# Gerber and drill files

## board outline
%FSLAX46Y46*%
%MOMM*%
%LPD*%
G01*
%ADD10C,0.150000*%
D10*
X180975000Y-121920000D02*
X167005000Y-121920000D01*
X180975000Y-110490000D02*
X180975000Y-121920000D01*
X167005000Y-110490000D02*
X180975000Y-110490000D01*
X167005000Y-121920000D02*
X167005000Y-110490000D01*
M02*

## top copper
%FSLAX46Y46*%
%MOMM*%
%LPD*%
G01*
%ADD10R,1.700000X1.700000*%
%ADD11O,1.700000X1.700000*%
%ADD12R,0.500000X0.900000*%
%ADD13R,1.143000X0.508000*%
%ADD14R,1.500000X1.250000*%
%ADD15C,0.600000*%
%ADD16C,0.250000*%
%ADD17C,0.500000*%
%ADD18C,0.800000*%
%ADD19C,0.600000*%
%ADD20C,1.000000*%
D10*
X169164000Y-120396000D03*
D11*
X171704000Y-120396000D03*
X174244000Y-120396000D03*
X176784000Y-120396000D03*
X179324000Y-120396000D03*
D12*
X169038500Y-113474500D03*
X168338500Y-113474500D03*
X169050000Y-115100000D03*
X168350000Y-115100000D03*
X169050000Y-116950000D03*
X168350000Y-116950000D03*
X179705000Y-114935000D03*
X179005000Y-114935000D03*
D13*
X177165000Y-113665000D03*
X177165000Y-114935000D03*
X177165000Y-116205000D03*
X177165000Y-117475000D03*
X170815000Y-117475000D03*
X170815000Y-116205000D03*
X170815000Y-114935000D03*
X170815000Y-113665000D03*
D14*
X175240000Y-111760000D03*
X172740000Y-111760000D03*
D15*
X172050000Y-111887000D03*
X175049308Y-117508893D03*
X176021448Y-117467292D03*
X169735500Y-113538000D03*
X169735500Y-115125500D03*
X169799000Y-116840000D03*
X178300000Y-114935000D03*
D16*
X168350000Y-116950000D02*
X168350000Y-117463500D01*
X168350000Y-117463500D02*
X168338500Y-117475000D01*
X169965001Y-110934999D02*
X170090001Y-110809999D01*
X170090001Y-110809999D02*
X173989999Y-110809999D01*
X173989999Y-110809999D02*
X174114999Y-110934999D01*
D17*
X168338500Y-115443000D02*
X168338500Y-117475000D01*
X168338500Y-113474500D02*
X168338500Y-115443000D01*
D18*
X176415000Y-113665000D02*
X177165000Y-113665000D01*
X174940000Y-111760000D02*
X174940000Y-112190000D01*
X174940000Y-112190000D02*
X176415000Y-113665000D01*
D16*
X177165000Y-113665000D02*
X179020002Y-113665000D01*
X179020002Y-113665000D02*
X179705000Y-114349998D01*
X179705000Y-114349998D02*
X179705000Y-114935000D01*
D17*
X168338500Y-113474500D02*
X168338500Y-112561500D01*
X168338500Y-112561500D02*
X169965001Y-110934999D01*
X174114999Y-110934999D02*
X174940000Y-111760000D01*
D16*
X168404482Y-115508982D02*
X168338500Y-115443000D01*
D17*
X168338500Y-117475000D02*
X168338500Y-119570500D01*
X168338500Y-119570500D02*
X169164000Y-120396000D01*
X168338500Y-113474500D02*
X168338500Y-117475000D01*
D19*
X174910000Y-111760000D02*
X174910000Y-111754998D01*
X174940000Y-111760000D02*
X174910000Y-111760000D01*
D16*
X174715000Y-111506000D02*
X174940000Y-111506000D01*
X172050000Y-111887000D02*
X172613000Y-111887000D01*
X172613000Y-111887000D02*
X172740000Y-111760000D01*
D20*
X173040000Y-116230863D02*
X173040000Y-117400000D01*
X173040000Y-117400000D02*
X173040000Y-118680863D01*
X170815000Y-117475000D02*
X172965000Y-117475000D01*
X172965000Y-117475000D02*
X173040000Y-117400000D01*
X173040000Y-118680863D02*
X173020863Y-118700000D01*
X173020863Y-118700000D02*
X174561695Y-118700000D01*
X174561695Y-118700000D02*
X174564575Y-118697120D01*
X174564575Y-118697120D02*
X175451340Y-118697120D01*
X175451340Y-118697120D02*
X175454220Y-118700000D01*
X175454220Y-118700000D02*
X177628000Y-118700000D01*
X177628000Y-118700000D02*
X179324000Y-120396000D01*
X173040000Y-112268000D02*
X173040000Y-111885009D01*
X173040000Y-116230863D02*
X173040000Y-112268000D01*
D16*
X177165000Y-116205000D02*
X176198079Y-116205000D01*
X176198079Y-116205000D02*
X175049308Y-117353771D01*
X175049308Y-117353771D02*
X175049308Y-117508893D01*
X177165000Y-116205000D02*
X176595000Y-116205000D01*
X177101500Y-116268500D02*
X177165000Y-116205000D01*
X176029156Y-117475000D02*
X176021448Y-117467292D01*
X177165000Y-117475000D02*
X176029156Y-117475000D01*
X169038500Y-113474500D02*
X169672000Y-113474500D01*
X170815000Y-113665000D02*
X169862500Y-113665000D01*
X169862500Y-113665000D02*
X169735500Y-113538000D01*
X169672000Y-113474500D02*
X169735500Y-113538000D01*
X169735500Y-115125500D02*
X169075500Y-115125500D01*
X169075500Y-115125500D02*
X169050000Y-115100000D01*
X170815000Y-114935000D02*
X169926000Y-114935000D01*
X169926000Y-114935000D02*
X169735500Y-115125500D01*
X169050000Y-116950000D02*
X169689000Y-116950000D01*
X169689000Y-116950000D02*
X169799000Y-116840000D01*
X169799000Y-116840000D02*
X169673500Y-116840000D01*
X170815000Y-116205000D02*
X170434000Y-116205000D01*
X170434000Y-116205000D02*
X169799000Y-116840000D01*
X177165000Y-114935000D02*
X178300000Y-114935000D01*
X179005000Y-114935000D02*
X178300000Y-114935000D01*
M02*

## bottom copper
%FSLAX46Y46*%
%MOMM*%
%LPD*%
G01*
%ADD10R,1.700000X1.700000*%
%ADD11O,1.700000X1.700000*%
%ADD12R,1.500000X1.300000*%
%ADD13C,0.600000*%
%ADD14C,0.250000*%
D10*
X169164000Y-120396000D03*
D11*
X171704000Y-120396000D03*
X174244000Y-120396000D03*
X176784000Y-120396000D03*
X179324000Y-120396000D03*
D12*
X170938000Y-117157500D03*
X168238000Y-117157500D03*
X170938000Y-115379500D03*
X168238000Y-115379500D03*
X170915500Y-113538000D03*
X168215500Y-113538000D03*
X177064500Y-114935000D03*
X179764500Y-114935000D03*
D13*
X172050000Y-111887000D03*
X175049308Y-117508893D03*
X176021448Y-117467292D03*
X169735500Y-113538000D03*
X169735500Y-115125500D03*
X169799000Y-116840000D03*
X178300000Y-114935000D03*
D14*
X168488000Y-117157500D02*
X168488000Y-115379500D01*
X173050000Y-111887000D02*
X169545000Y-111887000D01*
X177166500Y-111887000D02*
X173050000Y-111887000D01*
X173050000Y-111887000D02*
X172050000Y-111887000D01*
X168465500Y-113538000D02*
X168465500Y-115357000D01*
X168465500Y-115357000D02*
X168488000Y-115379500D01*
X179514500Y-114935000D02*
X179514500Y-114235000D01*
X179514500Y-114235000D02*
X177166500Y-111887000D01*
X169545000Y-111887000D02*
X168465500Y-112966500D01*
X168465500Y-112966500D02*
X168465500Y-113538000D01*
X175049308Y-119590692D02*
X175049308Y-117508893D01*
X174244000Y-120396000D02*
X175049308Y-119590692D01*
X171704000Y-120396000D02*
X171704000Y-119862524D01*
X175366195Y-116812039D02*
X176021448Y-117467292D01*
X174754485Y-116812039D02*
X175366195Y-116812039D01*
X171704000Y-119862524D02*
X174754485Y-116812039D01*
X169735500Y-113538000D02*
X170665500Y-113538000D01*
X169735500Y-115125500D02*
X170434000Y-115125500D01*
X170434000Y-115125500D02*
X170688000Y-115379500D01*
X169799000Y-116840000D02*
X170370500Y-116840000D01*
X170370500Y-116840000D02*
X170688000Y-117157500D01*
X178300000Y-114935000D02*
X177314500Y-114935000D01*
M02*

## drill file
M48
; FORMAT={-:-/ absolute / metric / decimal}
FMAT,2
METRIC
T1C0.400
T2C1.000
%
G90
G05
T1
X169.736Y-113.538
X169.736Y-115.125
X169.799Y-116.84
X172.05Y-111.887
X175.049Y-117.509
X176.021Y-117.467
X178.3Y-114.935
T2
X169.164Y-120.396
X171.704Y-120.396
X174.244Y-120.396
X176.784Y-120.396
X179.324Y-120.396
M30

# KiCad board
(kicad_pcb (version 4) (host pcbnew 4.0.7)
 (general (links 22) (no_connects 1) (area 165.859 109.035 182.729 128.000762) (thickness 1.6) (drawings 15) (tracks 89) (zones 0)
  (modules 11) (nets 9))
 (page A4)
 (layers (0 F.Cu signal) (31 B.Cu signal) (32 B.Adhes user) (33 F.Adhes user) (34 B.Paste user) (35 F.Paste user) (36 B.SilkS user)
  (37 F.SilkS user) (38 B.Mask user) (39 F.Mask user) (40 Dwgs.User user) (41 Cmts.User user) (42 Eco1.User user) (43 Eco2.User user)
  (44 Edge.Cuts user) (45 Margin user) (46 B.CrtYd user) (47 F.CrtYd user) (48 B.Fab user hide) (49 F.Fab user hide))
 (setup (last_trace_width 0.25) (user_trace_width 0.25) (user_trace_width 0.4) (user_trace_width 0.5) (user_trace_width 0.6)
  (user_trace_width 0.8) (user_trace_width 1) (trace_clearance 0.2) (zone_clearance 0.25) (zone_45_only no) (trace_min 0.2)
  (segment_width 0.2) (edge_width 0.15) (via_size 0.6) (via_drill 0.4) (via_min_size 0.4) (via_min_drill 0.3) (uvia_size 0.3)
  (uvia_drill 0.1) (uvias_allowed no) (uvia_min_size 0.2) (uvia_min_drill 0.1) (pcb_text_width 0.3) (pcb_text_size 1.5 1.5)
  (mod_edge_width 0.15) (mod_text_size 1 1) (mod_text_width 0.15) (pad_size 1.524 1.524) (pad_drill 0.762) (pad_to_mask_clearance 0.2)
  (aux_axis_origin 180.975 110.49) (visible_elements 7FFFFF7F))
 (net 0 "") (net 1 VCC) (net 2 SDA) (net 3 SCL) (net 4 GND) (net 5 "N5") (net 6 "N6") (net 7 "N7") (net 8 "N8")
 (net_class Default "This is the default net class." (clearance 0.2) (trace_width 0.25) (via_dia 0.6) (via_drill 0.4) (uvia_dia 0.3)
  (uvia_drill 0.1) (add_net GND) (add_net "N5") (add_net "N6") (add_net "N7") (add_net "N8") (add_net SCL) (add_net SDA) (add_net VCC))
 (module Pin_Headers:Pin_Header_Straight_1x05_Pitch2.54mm (layer F.Cu) (at 169.164 120.396 90)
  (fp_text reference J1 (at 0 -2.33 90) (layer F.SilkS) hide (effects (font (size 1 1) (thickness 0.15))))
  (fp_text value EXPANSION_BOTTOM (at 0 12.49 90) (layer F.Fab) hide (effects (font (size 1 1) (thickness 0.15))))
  (pad 1 thru_hole rect (at 0 0 90) (size 1.7 1.7) (drill 1) (layers *.Cu *.Mask) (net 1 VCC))
  (pad 2 thru_hole oval (at 0 2.54 90) (size 1.7 1.7) (drill 1) (layers *.Cu *.Mask) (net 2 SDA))
  (pad 3 thru_hole oval (at 0 5.08 90) (size 1.7 1.7) (drill 1) (layers *.Cu *.Mask) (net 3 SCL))
  (pad 4 thru_hole oval (at 0 7.62 90) (size 1.7 1.7) (drill 1) (layers *.Cu *.Mask))
  (pad 5 thru_hole oval (at 0 10.16 90) (size 1.7 1.7) (drill 1) (layers *.Cu *.Mask) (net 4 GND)))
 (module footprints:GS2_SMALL (layer F.Cu) (at 168.3385 113.4745 270)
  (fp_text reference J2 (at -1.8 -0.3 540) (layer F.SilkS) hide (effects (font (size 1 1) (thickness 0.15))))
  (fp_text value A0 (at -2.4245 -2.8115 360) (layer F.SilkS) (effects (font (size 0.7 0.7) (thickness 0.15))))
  (pad 1 smd rect (at 0 -0.7 270) (size 0.9 0.5) (layers F.Cu F.Paste F.Mask) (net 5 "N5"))
  (pad 2 smd rect (at 0 0 270) (size 0.9 0.5) (layers F.Cu F.Paste F.Mask) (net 1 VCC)))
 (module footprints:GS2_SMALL (layer F.Cu) (at 168.35 115.1 270)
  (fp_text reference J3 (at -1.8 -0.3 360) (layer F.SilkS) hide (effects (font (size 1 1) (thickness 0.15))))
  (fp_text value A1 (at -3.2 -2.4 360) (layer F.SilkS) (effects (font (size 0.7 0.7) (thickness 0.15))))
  (pad 1 smd rect (at 0 -0.7 270) (size 0.9 0.5) (layers F.Cu F.Paste F.Mask) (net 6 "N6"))
  (pad 2 smd rect (at 0 0 270) (size 0.9 0.5) (layers F.Cu F.Paste F.Mask) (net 1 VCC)))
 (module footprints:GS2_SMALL (layer F.Cu) (at 168.35 116.95 270)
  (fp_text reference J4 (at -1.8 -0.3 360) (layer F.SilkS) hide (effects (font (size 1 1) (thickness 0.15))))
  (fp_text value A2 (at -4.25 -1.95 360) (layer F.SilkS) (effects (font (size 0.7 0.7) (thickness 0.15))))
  (pad 1 smd rect (at 0 -0.7 270) (size 0.9 0.5) (layers F.Cu F.Paste F.Mask) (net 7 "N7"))
  (pad 2 smd rect (at 0 0 270) (size 0.9 0.5) (layers F.Cu F.Paste F.Mask) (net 1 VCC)))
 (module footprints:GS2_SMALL (layer F.Cu) (at 179.005 114.935 270)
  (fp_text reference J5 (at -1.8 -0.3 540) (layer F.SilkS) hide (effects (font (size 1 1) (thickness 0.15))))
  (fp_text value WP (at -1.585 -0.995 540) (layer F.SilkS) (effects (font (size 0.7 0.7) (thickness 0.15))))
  (pad 1 smd rect (at 0 -0.7 270) (size 0.9 0.5) (layers F.Cu F.Paste F.Mask) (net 1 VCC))
  (pad 2 smd rect (at 0 0 270) (size 0.9 0.5) (layers F.Cu F.Paste F.Mask) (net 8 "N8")))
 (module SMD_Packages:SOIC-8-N (layer F.Cu) (at 173.99 115.57 270)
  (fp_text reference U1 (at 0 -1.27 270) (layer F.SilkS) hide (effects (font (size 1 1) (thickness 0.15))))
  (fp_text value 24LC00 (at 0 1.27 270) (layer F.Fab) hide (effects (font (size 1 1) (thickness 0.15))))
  (pad 8 smd rect (at -1.905 -3.175 270) (size 0.508 1.143) (layers F.Cu F.Paste F.Mask) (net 1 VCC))
  (pad 7 smd rect (at -0.635 -3.175 270) (size 0.508 1.143) (layers F.Cu F.Paste F.Mask) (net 8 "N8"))
  (pad 6 smd rect (at 0.635 -3.175 270) (size 0.508 1.143) (layers F.Cu F.Paste F.Mask) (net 3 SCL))
  (pad 5 smd rect (at 1.905 -3.175 270) (size 0.508 1.143) (layers F.Cu F.Paste F.Mask) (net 2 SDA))
  (pad 4 smd rect (at 1.905 3.175 270) (size 0.508 1.143) (layers F.Cu F.Paste F.Mask) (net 4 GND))
  (pad 3 smd rect (at 0.635 3.175 270) (size 0.508 1.143) (layers F.Cu F.Paste F.Mask) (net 7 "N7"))
  (pad 2 smd rect (at -0.635 3.175 270) (size 0.508 1.143) (layers F.Cu F.Paste F.Mask) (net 6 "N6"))
  (pad 1 smd rect (at -1.905 3.175 270) (size 0.508 1.143) (layers F.Cu F.Paste F.Mask) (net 5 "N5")))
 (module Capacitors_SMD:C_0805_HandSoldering (layer F.Cu) (at 173.99 111.76 180)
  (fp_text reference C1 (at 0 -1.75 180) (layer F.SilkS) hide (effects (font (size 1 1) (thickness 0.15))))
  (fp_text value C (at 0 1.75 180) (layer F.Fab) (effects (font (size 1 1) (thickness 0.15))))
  (pad 1 smd rect (at -1.25 0 180) (size 1.5 1.25) (layers F.Cu F.Paste F.Mask) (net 1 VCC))
  (pad 2 smd rect (at 1.25 0 180) (size 1.5 1.25) (layers F.Cu F.Paste F.Mask) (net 4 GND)))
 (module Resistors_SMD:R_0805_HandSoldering (layer B.Cu) (at 169.588 117.1575 180)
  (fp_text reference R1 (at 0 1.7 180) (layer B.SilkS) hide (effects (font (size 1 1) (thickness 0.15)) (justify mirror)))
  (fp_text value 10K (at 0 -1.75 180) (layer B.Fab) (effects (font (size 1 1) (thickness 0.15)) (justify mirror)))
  (pad 1 smd rect (at -1.35 0 180) (size 1.5 1.3) (layers B.Cu B.Paste B.Mask) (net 7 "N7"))
  (pad 2 smd rect (at 1.35 0 180) (size 1.5 1.3) (layers B.Cu B.Paste B.Mask) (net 4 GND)))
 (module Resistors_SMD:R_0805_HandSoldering (layer B.Cu) (at 169.588 115.3795 180)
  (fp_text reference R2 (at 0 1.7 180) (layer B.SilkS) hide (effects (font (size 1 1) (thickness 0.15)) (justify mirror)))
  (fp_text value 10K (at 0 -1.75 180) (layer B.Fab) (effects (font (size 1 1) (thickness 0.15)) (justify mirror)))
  (pad 1 smd rect (at -1.35 0 180) (size 1.5 1.3) (layers B.Cu B.Paste B.Mask) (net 6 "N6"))
  (pad 2 smd rect (at 1.35 0 180) (size 1.5 1.3) (layers B.Cu B.Paste B.Mask) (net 4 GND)))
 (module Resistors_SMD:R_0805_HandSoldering (layer B.Cu) (at 169.5655 113.538 180)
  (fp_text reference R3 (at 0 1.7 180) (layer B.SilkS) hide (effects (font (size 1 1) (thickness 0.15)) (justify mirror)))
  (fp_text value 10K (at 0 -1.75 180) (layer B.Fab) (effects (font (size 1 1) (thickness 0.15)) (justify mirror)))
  (pad 1 smd rect (at -1.35 0 180) (size 1.5 1.3) (layers B.Cu B.Paste B.Mask) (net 5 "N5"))
  (pad 2 smd rect (at 1.35 0 180) (size 1.5 1.3) (layers B.Cu B.Paste B.Mask) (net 4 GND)))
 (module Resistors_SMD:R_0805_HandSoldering (layer B.Cu) (at 178.4145 114.935)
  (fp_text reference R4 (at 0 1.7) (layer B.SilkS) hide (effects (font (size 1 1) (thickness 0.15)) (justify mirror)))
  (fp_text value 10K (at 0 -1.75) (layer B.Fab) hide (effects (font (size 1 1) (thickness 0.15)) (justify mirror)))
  (pad 1 smd rect (at -1.35 0) (size 1.5 1.3) (layers B.Cu B.Paste B.Mask) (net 8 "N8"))
  (pad 2 smd rect (at 1.35 0) (size 1.5 1.3) (layers B.Cu B.Paste B.Mask) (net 4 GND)))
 (gr_line (start 180.975 121.92) (end 167.005 121.92) (layer Edge.Cuts) (width 0.15))
 (gr_line (start 180.975 110.49) (end 180.975 121.92) (layer Edge.Cuts) (width 0.15))
 (gr_line (start 167.005 110.49) (end 180.975 110.49) (layer Edge.Cuts) (width 0.15))
 (gr_line (start 167.005 121.92) (end 167.005 110.49) (layer Edge.Cuts) (width 0.15))
 (segment (start 168.35 116.95) (end 168.35 117.4635) (width 0.25) (layer F.Cu) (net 1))
 (segment (start 168.35 117.4635) (end 168.3385 117.475) (width 0.25) (layer F.Cu) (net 1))
 (segment (start 169.965001 110.934999) (end 170.090001 110.809999) (width 0.25) (layer F.Cu) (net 1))
 (segment (start 170.090001 110.809999) (end 173.989999 110.809999) (width 0.25) (layer F.Cu) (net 1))
 (segment (start 173.989999 110.809999) (end 174.114999 110.934999) (width 0.25) (layer F.Cu) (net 1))
 (segment (start 168.3385 115.443) (end 168.3385 117.475) (width 0.5) (layer F.Cu) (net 1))
 (segment (start 168.3385 113.4745) (end 168.3385 115.443) (width 0.5) (layer F.Cu) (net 1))
 (segment (start 176.415 113.665) (end 177.165 113.665) (width 0.8) (layer F.Cu) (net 1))
 (segment (start 174.94 111.76) (end 174.94 112.19) (width 0.8) (layer F.Cu) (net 1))
 (segment (start 174.94 112.19) (end 176.415 113.665) (width 0.8) (layer F.Cu) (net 1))
 (segment (start 177.165 113.665) (end 179.020002 113.665) (width 0.25) (layer F.Cu) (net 1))
 (segment (start 179.020002 113.665) (end 179.705 114.349998) (width 0.25) (layer F.Cu) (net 1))
 (segment (start 179.705 114.349998) (end 179.705 114.935) (width 0.25) (layer F.Cu) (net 1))
 (segment (start 168.3385 113.4745) (end 168.3385 112.5615) (width 0.5) (layer F.Cu) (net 1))
 (segment (start 168.3385 112.5615) (end 169.965001 110.934999) (width 0.5) (layer F.Cu) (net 1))
 (segment (start 174.114999 110.934999) (end 174.94 111.76) (width 0.5) (layer F.Cu) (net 1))
 (segment (start 168.404482 115.508982) (end 168.3385 115.443) (width 0.25) (layer F.Cu) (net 1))
 (segment (start 168.3385 117.475) (end 168.3385 119.5705) (width 0.5) (layer F.Cu) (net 1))
 (segment (start 168.3385 119.5705) (end 169.164 120.396) (width 0.5) (layer F.Cu) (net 1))
 (segment (start 168.3385 113.4745) (end 168.3385 117.475) (width 0.5) (layer F.Cu) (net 1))
 (segment (start 174.91 111.76) (end 174.91 111.754998) (width 0.6) (layer F.Cu) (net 1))
 (segment (start 174.94 111.76) (end 174.91 111.76) (width 0.6) (layer F.Cu) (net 1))
 (segment (start 174.715 111.506) (end 174.94 111.506) (width 0.25) (layer F.Cu) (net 1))
 (segment (start 172.05 111.887) (end 172.613 111.887) (width 0.25) (layer F.Cu) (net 4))
 (segment (start 172.613 111.887) (end 172.74 111.76) (width 0.25) (layer F.Cu) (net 4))
 (segment (start 173.04 116.230863) (end 173.04 117.4) (width 1) (layer F.Cu) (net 4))
 (segment (start 173.04 117.4) (end 173.04 118.680863) (width 1) (layer F.Cu) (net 4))
 (segment (start 170.815 117.475) (end 172.965 117.475) (width 1) (layer F.Cu) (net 4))
 (segment (start 172.965 117.475) (end 173.04 117.4) (width 1) (layer F.Cu) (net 4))
 (segment (start 173.04 118.680863) (end 173.020863 118.7) (width 1) (layer F.Cu) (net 4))
 (segment (start 173.020863 118.7) (end 174.561695 118.7) (width 1) (layer F.Cu) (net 4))
 (segment (start 174.561695 118.7) (end 174.564575 118.69712) (width 1) (layer F.Cu) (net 4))
 (segment (start 174.564575 118.69712) (end 175.45134 118.69712) (width 1) (layer F.Cu) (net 4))
 (segment (start 175.45134 118.69712) (end 175.45422 118.7) (width 1) (layer F.Cu) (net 4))
 (segment (start 175.45422 118.7) (end 177.628 118.7) (width 1) (layer F.Cu) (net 4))
 (segment (start 177.628 118.7) (end 179.324 120.396) (width 1) (layer F.Cu) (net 4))
 (segment (start 168.488 117.1575) (end 168.488 115.3795) (width 0.25) (layer B.Cu) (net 4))
 (segment (start 173.05 111.887) (end 169.545 111.887) (width 0.25) (layer B.Cu) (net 4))
 (segment (start 177.1665 111.887) (end 173.05 111.887) (width 0.25) (layer B.Cu) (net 4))
 (segment (start 173.05 111.887) (end 172.05 111.887) (width 0.25) (layer B.Cu) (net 4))
 (via (at 172.05 111.887) (size 0.6) (drill 0.4) (layers F.Cu B.Cu) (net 4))
 (segment (start 173.04 112.268) (end 173.04 111.885009) (width 1) (layer F.Cu) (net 4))
 (segment (start 173.04 116.230863) (end 173.04 112.268) (width 1) (layer F.Cu) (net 4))
 (segment (start 168.4655 113.538) (end 168.4655 115.357) (width 0.25) (layer B.Cu) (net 4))
 (segment (start 168.4655 115.357) (end 168.488 115.3795) (width 0.25) (layer B.Cu) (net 4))
 (segment (start 179.5145 114.935) (end 179.5145 114.235) (width 0.25) (layer B.Cu) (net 4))
 (segment (start 179.5145 114.235) (end 177.1665 111.887) (width 0.25) (layer B.Cu) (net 4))
 (segment (start 169.545 111.887) (end 168.4655 112.9665) (width 0.25) (layer B.Cu) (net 4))
 (segment (start 168.4655 112.9665) (end 168.4655 113.538) (width 0.25) (layer B.Cu) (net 4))
 (segment (start 177.165 116.205) (end 176.198079 116.205) (width 0.25) (layer F.Cu) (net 3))
 (segment (start 176.198079 116.205) (end 175.049308 117.353771) (width 0.25) (layer F.Cu) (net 3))
 (segment (start 175.049308 117.353771) (end 175.049308 117.508893) (width 0.25) (layer F.Cu) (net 3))
 (segment (start 175.049308 119.590692) (end 175.049308 117.508893) (width 0.25) (layer B.Cu) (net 3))
 (via (at 175.049308 117.508893) (size 0.6) (drill 0.4) (layers F.Cu B.Cu) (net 3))
 (segment (start 174.244 120.396) (end 175.049308 119.590692) (width 0.25) (layer B.Cu) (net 3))
 (segment (start 177.165 116.205) (end 176.595 116.205) (width 0.25) (layer F.Cu) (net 3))
 (segment (start 177.1015 116.2685) (end 177.165 116.205) (width 0.25) (layer F.Cu) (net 3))
 (segment (start 171.704 120.396) (end 171.704 119.862524) (width 0.25) (layer B.Cu) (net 2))
 (segment (start 176.029156 117.475) (end 176.021448 117.467292) (width 0.25) (layer F.Cu) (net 2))
 (segment (start 177.165 117.475) (end 176.029156 117.475) (width 0.25) (layer F.Cu) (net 2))
 (segment (start 175.366195 116.812039) (end 176.021448 117.467292) (width 0.25) (layer B.Cu) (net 2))
 (segment (start 174.754485 116.812039) (end 175.366195 116.812039) (width 0.25) (layer B.Cu) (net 2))
 (segment (start 171.704 119.862524) (end 174.754485 116.812039) (width 0.25) (layer B.Cu) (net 2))
 (via (at 176.021448 117.467292) (size 0.6) (drill 0.4) (layers F.Cu B.Cu) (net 2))
 (segment (start 169.0385 113.4745) (end 169.672 113.4745) (width 0.25) (layer F.Cu) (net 5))
 (segment (start 170.815 113.665) (end 169.8625 113.665) (width 0.25) (layer F.Cu) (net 5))
 (segment (start 169.8625 113.665) (end 169.7355 113.538) (width 0.25) (layer F.Cu) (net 5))
 (segment (start 169.7355 113.538) (end 170.6655 113.538) (width 0.25) (layer B.Cu) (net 5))
 (segment (start 169.672 113.4745) (end 169.7355 113.538) (width 0.25) (layer F.Cu) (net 5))
 (via (at 169.7355 113.538) (size 0.6) (drill 0.4) (layers F.Cu B.Cu) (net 5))
 (segment (start 169.7355 115.1255) (end 169.0755 115.1255) (width 0.25) (layer F.Cu) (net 6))
 (segment (start 169.0755 115.1255) (end 169.05 115.1) (width 0.25) (layer F.Cu) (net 6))
 (segment (start 169.7355 115.1255) (end 170.434 115.1255) (width 0.25) (layer B.Cu) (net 6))
 (segment (start 170.434 115.1255) (end 170.688 115.3795) (width 0.25) (layer B.Cu) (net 6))
 (segment (start 170.815 114.935) (end 169.926 114.935) (width 0.25) (layer F.Cu) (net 6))
 (segment (start 169.926 114.935) (end 169.7355 115.1255) (width 0.25) (layer F.Cu) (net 6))
 (via (at 169.7355 115.1255) (size 0.6) (drill 0.4) (layers F.Cu B.Cu) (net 6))
 (segment (start 169.05 116.95) (end 169.689 116.95) (width 0.25) (layer F.Cu) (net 7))
 (segment (start 169.689 116.95) (end 169.799 116.84) (width 0.25) (layer F.Cu) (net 7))
 (segment (start 169.799 116.84) (end 169.6735 116.84) (width 0.25) (layer F.Cu) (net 7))
 (segment (start 169.799 116.84) (end 170.3705 116.84) (width 0.25) (layer B.Cu) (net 7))
 (segment (start 170.3705 116.84) (end 170.688 117.1575) (width 0.25) (layer B.Cu) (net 7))
 (segment (start 170.815 116.205) (end 170.434 116.205) (width 0.25) (layer F.Cu) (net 7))
 (segment (start 170.434 116.205) (end 169.799 116.84) (width 0.25) (layer F.Cu) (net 7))
 (via (at 169.799 116.84) (size 0.6) (drill 0.4) (layers F.Cu B.Cu) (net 7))
 (segment (start 178.3 114.935) (end 177.3145 114.935) (width 0.25) (layer B.Cu) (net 8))
 (segment (start 177.165 114.935) (end 178.3 114.935) (width 0.25) (layer F.Cu) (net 8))
 (segment (start 179.005 114.935) (end 178.3 114.935) (width 0.25) (layer F.Cu) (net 8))
 (via (at 178.3 114.935) (size 0.6) (drill 0.4) (layers F.Cu B.Cu) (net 8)))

